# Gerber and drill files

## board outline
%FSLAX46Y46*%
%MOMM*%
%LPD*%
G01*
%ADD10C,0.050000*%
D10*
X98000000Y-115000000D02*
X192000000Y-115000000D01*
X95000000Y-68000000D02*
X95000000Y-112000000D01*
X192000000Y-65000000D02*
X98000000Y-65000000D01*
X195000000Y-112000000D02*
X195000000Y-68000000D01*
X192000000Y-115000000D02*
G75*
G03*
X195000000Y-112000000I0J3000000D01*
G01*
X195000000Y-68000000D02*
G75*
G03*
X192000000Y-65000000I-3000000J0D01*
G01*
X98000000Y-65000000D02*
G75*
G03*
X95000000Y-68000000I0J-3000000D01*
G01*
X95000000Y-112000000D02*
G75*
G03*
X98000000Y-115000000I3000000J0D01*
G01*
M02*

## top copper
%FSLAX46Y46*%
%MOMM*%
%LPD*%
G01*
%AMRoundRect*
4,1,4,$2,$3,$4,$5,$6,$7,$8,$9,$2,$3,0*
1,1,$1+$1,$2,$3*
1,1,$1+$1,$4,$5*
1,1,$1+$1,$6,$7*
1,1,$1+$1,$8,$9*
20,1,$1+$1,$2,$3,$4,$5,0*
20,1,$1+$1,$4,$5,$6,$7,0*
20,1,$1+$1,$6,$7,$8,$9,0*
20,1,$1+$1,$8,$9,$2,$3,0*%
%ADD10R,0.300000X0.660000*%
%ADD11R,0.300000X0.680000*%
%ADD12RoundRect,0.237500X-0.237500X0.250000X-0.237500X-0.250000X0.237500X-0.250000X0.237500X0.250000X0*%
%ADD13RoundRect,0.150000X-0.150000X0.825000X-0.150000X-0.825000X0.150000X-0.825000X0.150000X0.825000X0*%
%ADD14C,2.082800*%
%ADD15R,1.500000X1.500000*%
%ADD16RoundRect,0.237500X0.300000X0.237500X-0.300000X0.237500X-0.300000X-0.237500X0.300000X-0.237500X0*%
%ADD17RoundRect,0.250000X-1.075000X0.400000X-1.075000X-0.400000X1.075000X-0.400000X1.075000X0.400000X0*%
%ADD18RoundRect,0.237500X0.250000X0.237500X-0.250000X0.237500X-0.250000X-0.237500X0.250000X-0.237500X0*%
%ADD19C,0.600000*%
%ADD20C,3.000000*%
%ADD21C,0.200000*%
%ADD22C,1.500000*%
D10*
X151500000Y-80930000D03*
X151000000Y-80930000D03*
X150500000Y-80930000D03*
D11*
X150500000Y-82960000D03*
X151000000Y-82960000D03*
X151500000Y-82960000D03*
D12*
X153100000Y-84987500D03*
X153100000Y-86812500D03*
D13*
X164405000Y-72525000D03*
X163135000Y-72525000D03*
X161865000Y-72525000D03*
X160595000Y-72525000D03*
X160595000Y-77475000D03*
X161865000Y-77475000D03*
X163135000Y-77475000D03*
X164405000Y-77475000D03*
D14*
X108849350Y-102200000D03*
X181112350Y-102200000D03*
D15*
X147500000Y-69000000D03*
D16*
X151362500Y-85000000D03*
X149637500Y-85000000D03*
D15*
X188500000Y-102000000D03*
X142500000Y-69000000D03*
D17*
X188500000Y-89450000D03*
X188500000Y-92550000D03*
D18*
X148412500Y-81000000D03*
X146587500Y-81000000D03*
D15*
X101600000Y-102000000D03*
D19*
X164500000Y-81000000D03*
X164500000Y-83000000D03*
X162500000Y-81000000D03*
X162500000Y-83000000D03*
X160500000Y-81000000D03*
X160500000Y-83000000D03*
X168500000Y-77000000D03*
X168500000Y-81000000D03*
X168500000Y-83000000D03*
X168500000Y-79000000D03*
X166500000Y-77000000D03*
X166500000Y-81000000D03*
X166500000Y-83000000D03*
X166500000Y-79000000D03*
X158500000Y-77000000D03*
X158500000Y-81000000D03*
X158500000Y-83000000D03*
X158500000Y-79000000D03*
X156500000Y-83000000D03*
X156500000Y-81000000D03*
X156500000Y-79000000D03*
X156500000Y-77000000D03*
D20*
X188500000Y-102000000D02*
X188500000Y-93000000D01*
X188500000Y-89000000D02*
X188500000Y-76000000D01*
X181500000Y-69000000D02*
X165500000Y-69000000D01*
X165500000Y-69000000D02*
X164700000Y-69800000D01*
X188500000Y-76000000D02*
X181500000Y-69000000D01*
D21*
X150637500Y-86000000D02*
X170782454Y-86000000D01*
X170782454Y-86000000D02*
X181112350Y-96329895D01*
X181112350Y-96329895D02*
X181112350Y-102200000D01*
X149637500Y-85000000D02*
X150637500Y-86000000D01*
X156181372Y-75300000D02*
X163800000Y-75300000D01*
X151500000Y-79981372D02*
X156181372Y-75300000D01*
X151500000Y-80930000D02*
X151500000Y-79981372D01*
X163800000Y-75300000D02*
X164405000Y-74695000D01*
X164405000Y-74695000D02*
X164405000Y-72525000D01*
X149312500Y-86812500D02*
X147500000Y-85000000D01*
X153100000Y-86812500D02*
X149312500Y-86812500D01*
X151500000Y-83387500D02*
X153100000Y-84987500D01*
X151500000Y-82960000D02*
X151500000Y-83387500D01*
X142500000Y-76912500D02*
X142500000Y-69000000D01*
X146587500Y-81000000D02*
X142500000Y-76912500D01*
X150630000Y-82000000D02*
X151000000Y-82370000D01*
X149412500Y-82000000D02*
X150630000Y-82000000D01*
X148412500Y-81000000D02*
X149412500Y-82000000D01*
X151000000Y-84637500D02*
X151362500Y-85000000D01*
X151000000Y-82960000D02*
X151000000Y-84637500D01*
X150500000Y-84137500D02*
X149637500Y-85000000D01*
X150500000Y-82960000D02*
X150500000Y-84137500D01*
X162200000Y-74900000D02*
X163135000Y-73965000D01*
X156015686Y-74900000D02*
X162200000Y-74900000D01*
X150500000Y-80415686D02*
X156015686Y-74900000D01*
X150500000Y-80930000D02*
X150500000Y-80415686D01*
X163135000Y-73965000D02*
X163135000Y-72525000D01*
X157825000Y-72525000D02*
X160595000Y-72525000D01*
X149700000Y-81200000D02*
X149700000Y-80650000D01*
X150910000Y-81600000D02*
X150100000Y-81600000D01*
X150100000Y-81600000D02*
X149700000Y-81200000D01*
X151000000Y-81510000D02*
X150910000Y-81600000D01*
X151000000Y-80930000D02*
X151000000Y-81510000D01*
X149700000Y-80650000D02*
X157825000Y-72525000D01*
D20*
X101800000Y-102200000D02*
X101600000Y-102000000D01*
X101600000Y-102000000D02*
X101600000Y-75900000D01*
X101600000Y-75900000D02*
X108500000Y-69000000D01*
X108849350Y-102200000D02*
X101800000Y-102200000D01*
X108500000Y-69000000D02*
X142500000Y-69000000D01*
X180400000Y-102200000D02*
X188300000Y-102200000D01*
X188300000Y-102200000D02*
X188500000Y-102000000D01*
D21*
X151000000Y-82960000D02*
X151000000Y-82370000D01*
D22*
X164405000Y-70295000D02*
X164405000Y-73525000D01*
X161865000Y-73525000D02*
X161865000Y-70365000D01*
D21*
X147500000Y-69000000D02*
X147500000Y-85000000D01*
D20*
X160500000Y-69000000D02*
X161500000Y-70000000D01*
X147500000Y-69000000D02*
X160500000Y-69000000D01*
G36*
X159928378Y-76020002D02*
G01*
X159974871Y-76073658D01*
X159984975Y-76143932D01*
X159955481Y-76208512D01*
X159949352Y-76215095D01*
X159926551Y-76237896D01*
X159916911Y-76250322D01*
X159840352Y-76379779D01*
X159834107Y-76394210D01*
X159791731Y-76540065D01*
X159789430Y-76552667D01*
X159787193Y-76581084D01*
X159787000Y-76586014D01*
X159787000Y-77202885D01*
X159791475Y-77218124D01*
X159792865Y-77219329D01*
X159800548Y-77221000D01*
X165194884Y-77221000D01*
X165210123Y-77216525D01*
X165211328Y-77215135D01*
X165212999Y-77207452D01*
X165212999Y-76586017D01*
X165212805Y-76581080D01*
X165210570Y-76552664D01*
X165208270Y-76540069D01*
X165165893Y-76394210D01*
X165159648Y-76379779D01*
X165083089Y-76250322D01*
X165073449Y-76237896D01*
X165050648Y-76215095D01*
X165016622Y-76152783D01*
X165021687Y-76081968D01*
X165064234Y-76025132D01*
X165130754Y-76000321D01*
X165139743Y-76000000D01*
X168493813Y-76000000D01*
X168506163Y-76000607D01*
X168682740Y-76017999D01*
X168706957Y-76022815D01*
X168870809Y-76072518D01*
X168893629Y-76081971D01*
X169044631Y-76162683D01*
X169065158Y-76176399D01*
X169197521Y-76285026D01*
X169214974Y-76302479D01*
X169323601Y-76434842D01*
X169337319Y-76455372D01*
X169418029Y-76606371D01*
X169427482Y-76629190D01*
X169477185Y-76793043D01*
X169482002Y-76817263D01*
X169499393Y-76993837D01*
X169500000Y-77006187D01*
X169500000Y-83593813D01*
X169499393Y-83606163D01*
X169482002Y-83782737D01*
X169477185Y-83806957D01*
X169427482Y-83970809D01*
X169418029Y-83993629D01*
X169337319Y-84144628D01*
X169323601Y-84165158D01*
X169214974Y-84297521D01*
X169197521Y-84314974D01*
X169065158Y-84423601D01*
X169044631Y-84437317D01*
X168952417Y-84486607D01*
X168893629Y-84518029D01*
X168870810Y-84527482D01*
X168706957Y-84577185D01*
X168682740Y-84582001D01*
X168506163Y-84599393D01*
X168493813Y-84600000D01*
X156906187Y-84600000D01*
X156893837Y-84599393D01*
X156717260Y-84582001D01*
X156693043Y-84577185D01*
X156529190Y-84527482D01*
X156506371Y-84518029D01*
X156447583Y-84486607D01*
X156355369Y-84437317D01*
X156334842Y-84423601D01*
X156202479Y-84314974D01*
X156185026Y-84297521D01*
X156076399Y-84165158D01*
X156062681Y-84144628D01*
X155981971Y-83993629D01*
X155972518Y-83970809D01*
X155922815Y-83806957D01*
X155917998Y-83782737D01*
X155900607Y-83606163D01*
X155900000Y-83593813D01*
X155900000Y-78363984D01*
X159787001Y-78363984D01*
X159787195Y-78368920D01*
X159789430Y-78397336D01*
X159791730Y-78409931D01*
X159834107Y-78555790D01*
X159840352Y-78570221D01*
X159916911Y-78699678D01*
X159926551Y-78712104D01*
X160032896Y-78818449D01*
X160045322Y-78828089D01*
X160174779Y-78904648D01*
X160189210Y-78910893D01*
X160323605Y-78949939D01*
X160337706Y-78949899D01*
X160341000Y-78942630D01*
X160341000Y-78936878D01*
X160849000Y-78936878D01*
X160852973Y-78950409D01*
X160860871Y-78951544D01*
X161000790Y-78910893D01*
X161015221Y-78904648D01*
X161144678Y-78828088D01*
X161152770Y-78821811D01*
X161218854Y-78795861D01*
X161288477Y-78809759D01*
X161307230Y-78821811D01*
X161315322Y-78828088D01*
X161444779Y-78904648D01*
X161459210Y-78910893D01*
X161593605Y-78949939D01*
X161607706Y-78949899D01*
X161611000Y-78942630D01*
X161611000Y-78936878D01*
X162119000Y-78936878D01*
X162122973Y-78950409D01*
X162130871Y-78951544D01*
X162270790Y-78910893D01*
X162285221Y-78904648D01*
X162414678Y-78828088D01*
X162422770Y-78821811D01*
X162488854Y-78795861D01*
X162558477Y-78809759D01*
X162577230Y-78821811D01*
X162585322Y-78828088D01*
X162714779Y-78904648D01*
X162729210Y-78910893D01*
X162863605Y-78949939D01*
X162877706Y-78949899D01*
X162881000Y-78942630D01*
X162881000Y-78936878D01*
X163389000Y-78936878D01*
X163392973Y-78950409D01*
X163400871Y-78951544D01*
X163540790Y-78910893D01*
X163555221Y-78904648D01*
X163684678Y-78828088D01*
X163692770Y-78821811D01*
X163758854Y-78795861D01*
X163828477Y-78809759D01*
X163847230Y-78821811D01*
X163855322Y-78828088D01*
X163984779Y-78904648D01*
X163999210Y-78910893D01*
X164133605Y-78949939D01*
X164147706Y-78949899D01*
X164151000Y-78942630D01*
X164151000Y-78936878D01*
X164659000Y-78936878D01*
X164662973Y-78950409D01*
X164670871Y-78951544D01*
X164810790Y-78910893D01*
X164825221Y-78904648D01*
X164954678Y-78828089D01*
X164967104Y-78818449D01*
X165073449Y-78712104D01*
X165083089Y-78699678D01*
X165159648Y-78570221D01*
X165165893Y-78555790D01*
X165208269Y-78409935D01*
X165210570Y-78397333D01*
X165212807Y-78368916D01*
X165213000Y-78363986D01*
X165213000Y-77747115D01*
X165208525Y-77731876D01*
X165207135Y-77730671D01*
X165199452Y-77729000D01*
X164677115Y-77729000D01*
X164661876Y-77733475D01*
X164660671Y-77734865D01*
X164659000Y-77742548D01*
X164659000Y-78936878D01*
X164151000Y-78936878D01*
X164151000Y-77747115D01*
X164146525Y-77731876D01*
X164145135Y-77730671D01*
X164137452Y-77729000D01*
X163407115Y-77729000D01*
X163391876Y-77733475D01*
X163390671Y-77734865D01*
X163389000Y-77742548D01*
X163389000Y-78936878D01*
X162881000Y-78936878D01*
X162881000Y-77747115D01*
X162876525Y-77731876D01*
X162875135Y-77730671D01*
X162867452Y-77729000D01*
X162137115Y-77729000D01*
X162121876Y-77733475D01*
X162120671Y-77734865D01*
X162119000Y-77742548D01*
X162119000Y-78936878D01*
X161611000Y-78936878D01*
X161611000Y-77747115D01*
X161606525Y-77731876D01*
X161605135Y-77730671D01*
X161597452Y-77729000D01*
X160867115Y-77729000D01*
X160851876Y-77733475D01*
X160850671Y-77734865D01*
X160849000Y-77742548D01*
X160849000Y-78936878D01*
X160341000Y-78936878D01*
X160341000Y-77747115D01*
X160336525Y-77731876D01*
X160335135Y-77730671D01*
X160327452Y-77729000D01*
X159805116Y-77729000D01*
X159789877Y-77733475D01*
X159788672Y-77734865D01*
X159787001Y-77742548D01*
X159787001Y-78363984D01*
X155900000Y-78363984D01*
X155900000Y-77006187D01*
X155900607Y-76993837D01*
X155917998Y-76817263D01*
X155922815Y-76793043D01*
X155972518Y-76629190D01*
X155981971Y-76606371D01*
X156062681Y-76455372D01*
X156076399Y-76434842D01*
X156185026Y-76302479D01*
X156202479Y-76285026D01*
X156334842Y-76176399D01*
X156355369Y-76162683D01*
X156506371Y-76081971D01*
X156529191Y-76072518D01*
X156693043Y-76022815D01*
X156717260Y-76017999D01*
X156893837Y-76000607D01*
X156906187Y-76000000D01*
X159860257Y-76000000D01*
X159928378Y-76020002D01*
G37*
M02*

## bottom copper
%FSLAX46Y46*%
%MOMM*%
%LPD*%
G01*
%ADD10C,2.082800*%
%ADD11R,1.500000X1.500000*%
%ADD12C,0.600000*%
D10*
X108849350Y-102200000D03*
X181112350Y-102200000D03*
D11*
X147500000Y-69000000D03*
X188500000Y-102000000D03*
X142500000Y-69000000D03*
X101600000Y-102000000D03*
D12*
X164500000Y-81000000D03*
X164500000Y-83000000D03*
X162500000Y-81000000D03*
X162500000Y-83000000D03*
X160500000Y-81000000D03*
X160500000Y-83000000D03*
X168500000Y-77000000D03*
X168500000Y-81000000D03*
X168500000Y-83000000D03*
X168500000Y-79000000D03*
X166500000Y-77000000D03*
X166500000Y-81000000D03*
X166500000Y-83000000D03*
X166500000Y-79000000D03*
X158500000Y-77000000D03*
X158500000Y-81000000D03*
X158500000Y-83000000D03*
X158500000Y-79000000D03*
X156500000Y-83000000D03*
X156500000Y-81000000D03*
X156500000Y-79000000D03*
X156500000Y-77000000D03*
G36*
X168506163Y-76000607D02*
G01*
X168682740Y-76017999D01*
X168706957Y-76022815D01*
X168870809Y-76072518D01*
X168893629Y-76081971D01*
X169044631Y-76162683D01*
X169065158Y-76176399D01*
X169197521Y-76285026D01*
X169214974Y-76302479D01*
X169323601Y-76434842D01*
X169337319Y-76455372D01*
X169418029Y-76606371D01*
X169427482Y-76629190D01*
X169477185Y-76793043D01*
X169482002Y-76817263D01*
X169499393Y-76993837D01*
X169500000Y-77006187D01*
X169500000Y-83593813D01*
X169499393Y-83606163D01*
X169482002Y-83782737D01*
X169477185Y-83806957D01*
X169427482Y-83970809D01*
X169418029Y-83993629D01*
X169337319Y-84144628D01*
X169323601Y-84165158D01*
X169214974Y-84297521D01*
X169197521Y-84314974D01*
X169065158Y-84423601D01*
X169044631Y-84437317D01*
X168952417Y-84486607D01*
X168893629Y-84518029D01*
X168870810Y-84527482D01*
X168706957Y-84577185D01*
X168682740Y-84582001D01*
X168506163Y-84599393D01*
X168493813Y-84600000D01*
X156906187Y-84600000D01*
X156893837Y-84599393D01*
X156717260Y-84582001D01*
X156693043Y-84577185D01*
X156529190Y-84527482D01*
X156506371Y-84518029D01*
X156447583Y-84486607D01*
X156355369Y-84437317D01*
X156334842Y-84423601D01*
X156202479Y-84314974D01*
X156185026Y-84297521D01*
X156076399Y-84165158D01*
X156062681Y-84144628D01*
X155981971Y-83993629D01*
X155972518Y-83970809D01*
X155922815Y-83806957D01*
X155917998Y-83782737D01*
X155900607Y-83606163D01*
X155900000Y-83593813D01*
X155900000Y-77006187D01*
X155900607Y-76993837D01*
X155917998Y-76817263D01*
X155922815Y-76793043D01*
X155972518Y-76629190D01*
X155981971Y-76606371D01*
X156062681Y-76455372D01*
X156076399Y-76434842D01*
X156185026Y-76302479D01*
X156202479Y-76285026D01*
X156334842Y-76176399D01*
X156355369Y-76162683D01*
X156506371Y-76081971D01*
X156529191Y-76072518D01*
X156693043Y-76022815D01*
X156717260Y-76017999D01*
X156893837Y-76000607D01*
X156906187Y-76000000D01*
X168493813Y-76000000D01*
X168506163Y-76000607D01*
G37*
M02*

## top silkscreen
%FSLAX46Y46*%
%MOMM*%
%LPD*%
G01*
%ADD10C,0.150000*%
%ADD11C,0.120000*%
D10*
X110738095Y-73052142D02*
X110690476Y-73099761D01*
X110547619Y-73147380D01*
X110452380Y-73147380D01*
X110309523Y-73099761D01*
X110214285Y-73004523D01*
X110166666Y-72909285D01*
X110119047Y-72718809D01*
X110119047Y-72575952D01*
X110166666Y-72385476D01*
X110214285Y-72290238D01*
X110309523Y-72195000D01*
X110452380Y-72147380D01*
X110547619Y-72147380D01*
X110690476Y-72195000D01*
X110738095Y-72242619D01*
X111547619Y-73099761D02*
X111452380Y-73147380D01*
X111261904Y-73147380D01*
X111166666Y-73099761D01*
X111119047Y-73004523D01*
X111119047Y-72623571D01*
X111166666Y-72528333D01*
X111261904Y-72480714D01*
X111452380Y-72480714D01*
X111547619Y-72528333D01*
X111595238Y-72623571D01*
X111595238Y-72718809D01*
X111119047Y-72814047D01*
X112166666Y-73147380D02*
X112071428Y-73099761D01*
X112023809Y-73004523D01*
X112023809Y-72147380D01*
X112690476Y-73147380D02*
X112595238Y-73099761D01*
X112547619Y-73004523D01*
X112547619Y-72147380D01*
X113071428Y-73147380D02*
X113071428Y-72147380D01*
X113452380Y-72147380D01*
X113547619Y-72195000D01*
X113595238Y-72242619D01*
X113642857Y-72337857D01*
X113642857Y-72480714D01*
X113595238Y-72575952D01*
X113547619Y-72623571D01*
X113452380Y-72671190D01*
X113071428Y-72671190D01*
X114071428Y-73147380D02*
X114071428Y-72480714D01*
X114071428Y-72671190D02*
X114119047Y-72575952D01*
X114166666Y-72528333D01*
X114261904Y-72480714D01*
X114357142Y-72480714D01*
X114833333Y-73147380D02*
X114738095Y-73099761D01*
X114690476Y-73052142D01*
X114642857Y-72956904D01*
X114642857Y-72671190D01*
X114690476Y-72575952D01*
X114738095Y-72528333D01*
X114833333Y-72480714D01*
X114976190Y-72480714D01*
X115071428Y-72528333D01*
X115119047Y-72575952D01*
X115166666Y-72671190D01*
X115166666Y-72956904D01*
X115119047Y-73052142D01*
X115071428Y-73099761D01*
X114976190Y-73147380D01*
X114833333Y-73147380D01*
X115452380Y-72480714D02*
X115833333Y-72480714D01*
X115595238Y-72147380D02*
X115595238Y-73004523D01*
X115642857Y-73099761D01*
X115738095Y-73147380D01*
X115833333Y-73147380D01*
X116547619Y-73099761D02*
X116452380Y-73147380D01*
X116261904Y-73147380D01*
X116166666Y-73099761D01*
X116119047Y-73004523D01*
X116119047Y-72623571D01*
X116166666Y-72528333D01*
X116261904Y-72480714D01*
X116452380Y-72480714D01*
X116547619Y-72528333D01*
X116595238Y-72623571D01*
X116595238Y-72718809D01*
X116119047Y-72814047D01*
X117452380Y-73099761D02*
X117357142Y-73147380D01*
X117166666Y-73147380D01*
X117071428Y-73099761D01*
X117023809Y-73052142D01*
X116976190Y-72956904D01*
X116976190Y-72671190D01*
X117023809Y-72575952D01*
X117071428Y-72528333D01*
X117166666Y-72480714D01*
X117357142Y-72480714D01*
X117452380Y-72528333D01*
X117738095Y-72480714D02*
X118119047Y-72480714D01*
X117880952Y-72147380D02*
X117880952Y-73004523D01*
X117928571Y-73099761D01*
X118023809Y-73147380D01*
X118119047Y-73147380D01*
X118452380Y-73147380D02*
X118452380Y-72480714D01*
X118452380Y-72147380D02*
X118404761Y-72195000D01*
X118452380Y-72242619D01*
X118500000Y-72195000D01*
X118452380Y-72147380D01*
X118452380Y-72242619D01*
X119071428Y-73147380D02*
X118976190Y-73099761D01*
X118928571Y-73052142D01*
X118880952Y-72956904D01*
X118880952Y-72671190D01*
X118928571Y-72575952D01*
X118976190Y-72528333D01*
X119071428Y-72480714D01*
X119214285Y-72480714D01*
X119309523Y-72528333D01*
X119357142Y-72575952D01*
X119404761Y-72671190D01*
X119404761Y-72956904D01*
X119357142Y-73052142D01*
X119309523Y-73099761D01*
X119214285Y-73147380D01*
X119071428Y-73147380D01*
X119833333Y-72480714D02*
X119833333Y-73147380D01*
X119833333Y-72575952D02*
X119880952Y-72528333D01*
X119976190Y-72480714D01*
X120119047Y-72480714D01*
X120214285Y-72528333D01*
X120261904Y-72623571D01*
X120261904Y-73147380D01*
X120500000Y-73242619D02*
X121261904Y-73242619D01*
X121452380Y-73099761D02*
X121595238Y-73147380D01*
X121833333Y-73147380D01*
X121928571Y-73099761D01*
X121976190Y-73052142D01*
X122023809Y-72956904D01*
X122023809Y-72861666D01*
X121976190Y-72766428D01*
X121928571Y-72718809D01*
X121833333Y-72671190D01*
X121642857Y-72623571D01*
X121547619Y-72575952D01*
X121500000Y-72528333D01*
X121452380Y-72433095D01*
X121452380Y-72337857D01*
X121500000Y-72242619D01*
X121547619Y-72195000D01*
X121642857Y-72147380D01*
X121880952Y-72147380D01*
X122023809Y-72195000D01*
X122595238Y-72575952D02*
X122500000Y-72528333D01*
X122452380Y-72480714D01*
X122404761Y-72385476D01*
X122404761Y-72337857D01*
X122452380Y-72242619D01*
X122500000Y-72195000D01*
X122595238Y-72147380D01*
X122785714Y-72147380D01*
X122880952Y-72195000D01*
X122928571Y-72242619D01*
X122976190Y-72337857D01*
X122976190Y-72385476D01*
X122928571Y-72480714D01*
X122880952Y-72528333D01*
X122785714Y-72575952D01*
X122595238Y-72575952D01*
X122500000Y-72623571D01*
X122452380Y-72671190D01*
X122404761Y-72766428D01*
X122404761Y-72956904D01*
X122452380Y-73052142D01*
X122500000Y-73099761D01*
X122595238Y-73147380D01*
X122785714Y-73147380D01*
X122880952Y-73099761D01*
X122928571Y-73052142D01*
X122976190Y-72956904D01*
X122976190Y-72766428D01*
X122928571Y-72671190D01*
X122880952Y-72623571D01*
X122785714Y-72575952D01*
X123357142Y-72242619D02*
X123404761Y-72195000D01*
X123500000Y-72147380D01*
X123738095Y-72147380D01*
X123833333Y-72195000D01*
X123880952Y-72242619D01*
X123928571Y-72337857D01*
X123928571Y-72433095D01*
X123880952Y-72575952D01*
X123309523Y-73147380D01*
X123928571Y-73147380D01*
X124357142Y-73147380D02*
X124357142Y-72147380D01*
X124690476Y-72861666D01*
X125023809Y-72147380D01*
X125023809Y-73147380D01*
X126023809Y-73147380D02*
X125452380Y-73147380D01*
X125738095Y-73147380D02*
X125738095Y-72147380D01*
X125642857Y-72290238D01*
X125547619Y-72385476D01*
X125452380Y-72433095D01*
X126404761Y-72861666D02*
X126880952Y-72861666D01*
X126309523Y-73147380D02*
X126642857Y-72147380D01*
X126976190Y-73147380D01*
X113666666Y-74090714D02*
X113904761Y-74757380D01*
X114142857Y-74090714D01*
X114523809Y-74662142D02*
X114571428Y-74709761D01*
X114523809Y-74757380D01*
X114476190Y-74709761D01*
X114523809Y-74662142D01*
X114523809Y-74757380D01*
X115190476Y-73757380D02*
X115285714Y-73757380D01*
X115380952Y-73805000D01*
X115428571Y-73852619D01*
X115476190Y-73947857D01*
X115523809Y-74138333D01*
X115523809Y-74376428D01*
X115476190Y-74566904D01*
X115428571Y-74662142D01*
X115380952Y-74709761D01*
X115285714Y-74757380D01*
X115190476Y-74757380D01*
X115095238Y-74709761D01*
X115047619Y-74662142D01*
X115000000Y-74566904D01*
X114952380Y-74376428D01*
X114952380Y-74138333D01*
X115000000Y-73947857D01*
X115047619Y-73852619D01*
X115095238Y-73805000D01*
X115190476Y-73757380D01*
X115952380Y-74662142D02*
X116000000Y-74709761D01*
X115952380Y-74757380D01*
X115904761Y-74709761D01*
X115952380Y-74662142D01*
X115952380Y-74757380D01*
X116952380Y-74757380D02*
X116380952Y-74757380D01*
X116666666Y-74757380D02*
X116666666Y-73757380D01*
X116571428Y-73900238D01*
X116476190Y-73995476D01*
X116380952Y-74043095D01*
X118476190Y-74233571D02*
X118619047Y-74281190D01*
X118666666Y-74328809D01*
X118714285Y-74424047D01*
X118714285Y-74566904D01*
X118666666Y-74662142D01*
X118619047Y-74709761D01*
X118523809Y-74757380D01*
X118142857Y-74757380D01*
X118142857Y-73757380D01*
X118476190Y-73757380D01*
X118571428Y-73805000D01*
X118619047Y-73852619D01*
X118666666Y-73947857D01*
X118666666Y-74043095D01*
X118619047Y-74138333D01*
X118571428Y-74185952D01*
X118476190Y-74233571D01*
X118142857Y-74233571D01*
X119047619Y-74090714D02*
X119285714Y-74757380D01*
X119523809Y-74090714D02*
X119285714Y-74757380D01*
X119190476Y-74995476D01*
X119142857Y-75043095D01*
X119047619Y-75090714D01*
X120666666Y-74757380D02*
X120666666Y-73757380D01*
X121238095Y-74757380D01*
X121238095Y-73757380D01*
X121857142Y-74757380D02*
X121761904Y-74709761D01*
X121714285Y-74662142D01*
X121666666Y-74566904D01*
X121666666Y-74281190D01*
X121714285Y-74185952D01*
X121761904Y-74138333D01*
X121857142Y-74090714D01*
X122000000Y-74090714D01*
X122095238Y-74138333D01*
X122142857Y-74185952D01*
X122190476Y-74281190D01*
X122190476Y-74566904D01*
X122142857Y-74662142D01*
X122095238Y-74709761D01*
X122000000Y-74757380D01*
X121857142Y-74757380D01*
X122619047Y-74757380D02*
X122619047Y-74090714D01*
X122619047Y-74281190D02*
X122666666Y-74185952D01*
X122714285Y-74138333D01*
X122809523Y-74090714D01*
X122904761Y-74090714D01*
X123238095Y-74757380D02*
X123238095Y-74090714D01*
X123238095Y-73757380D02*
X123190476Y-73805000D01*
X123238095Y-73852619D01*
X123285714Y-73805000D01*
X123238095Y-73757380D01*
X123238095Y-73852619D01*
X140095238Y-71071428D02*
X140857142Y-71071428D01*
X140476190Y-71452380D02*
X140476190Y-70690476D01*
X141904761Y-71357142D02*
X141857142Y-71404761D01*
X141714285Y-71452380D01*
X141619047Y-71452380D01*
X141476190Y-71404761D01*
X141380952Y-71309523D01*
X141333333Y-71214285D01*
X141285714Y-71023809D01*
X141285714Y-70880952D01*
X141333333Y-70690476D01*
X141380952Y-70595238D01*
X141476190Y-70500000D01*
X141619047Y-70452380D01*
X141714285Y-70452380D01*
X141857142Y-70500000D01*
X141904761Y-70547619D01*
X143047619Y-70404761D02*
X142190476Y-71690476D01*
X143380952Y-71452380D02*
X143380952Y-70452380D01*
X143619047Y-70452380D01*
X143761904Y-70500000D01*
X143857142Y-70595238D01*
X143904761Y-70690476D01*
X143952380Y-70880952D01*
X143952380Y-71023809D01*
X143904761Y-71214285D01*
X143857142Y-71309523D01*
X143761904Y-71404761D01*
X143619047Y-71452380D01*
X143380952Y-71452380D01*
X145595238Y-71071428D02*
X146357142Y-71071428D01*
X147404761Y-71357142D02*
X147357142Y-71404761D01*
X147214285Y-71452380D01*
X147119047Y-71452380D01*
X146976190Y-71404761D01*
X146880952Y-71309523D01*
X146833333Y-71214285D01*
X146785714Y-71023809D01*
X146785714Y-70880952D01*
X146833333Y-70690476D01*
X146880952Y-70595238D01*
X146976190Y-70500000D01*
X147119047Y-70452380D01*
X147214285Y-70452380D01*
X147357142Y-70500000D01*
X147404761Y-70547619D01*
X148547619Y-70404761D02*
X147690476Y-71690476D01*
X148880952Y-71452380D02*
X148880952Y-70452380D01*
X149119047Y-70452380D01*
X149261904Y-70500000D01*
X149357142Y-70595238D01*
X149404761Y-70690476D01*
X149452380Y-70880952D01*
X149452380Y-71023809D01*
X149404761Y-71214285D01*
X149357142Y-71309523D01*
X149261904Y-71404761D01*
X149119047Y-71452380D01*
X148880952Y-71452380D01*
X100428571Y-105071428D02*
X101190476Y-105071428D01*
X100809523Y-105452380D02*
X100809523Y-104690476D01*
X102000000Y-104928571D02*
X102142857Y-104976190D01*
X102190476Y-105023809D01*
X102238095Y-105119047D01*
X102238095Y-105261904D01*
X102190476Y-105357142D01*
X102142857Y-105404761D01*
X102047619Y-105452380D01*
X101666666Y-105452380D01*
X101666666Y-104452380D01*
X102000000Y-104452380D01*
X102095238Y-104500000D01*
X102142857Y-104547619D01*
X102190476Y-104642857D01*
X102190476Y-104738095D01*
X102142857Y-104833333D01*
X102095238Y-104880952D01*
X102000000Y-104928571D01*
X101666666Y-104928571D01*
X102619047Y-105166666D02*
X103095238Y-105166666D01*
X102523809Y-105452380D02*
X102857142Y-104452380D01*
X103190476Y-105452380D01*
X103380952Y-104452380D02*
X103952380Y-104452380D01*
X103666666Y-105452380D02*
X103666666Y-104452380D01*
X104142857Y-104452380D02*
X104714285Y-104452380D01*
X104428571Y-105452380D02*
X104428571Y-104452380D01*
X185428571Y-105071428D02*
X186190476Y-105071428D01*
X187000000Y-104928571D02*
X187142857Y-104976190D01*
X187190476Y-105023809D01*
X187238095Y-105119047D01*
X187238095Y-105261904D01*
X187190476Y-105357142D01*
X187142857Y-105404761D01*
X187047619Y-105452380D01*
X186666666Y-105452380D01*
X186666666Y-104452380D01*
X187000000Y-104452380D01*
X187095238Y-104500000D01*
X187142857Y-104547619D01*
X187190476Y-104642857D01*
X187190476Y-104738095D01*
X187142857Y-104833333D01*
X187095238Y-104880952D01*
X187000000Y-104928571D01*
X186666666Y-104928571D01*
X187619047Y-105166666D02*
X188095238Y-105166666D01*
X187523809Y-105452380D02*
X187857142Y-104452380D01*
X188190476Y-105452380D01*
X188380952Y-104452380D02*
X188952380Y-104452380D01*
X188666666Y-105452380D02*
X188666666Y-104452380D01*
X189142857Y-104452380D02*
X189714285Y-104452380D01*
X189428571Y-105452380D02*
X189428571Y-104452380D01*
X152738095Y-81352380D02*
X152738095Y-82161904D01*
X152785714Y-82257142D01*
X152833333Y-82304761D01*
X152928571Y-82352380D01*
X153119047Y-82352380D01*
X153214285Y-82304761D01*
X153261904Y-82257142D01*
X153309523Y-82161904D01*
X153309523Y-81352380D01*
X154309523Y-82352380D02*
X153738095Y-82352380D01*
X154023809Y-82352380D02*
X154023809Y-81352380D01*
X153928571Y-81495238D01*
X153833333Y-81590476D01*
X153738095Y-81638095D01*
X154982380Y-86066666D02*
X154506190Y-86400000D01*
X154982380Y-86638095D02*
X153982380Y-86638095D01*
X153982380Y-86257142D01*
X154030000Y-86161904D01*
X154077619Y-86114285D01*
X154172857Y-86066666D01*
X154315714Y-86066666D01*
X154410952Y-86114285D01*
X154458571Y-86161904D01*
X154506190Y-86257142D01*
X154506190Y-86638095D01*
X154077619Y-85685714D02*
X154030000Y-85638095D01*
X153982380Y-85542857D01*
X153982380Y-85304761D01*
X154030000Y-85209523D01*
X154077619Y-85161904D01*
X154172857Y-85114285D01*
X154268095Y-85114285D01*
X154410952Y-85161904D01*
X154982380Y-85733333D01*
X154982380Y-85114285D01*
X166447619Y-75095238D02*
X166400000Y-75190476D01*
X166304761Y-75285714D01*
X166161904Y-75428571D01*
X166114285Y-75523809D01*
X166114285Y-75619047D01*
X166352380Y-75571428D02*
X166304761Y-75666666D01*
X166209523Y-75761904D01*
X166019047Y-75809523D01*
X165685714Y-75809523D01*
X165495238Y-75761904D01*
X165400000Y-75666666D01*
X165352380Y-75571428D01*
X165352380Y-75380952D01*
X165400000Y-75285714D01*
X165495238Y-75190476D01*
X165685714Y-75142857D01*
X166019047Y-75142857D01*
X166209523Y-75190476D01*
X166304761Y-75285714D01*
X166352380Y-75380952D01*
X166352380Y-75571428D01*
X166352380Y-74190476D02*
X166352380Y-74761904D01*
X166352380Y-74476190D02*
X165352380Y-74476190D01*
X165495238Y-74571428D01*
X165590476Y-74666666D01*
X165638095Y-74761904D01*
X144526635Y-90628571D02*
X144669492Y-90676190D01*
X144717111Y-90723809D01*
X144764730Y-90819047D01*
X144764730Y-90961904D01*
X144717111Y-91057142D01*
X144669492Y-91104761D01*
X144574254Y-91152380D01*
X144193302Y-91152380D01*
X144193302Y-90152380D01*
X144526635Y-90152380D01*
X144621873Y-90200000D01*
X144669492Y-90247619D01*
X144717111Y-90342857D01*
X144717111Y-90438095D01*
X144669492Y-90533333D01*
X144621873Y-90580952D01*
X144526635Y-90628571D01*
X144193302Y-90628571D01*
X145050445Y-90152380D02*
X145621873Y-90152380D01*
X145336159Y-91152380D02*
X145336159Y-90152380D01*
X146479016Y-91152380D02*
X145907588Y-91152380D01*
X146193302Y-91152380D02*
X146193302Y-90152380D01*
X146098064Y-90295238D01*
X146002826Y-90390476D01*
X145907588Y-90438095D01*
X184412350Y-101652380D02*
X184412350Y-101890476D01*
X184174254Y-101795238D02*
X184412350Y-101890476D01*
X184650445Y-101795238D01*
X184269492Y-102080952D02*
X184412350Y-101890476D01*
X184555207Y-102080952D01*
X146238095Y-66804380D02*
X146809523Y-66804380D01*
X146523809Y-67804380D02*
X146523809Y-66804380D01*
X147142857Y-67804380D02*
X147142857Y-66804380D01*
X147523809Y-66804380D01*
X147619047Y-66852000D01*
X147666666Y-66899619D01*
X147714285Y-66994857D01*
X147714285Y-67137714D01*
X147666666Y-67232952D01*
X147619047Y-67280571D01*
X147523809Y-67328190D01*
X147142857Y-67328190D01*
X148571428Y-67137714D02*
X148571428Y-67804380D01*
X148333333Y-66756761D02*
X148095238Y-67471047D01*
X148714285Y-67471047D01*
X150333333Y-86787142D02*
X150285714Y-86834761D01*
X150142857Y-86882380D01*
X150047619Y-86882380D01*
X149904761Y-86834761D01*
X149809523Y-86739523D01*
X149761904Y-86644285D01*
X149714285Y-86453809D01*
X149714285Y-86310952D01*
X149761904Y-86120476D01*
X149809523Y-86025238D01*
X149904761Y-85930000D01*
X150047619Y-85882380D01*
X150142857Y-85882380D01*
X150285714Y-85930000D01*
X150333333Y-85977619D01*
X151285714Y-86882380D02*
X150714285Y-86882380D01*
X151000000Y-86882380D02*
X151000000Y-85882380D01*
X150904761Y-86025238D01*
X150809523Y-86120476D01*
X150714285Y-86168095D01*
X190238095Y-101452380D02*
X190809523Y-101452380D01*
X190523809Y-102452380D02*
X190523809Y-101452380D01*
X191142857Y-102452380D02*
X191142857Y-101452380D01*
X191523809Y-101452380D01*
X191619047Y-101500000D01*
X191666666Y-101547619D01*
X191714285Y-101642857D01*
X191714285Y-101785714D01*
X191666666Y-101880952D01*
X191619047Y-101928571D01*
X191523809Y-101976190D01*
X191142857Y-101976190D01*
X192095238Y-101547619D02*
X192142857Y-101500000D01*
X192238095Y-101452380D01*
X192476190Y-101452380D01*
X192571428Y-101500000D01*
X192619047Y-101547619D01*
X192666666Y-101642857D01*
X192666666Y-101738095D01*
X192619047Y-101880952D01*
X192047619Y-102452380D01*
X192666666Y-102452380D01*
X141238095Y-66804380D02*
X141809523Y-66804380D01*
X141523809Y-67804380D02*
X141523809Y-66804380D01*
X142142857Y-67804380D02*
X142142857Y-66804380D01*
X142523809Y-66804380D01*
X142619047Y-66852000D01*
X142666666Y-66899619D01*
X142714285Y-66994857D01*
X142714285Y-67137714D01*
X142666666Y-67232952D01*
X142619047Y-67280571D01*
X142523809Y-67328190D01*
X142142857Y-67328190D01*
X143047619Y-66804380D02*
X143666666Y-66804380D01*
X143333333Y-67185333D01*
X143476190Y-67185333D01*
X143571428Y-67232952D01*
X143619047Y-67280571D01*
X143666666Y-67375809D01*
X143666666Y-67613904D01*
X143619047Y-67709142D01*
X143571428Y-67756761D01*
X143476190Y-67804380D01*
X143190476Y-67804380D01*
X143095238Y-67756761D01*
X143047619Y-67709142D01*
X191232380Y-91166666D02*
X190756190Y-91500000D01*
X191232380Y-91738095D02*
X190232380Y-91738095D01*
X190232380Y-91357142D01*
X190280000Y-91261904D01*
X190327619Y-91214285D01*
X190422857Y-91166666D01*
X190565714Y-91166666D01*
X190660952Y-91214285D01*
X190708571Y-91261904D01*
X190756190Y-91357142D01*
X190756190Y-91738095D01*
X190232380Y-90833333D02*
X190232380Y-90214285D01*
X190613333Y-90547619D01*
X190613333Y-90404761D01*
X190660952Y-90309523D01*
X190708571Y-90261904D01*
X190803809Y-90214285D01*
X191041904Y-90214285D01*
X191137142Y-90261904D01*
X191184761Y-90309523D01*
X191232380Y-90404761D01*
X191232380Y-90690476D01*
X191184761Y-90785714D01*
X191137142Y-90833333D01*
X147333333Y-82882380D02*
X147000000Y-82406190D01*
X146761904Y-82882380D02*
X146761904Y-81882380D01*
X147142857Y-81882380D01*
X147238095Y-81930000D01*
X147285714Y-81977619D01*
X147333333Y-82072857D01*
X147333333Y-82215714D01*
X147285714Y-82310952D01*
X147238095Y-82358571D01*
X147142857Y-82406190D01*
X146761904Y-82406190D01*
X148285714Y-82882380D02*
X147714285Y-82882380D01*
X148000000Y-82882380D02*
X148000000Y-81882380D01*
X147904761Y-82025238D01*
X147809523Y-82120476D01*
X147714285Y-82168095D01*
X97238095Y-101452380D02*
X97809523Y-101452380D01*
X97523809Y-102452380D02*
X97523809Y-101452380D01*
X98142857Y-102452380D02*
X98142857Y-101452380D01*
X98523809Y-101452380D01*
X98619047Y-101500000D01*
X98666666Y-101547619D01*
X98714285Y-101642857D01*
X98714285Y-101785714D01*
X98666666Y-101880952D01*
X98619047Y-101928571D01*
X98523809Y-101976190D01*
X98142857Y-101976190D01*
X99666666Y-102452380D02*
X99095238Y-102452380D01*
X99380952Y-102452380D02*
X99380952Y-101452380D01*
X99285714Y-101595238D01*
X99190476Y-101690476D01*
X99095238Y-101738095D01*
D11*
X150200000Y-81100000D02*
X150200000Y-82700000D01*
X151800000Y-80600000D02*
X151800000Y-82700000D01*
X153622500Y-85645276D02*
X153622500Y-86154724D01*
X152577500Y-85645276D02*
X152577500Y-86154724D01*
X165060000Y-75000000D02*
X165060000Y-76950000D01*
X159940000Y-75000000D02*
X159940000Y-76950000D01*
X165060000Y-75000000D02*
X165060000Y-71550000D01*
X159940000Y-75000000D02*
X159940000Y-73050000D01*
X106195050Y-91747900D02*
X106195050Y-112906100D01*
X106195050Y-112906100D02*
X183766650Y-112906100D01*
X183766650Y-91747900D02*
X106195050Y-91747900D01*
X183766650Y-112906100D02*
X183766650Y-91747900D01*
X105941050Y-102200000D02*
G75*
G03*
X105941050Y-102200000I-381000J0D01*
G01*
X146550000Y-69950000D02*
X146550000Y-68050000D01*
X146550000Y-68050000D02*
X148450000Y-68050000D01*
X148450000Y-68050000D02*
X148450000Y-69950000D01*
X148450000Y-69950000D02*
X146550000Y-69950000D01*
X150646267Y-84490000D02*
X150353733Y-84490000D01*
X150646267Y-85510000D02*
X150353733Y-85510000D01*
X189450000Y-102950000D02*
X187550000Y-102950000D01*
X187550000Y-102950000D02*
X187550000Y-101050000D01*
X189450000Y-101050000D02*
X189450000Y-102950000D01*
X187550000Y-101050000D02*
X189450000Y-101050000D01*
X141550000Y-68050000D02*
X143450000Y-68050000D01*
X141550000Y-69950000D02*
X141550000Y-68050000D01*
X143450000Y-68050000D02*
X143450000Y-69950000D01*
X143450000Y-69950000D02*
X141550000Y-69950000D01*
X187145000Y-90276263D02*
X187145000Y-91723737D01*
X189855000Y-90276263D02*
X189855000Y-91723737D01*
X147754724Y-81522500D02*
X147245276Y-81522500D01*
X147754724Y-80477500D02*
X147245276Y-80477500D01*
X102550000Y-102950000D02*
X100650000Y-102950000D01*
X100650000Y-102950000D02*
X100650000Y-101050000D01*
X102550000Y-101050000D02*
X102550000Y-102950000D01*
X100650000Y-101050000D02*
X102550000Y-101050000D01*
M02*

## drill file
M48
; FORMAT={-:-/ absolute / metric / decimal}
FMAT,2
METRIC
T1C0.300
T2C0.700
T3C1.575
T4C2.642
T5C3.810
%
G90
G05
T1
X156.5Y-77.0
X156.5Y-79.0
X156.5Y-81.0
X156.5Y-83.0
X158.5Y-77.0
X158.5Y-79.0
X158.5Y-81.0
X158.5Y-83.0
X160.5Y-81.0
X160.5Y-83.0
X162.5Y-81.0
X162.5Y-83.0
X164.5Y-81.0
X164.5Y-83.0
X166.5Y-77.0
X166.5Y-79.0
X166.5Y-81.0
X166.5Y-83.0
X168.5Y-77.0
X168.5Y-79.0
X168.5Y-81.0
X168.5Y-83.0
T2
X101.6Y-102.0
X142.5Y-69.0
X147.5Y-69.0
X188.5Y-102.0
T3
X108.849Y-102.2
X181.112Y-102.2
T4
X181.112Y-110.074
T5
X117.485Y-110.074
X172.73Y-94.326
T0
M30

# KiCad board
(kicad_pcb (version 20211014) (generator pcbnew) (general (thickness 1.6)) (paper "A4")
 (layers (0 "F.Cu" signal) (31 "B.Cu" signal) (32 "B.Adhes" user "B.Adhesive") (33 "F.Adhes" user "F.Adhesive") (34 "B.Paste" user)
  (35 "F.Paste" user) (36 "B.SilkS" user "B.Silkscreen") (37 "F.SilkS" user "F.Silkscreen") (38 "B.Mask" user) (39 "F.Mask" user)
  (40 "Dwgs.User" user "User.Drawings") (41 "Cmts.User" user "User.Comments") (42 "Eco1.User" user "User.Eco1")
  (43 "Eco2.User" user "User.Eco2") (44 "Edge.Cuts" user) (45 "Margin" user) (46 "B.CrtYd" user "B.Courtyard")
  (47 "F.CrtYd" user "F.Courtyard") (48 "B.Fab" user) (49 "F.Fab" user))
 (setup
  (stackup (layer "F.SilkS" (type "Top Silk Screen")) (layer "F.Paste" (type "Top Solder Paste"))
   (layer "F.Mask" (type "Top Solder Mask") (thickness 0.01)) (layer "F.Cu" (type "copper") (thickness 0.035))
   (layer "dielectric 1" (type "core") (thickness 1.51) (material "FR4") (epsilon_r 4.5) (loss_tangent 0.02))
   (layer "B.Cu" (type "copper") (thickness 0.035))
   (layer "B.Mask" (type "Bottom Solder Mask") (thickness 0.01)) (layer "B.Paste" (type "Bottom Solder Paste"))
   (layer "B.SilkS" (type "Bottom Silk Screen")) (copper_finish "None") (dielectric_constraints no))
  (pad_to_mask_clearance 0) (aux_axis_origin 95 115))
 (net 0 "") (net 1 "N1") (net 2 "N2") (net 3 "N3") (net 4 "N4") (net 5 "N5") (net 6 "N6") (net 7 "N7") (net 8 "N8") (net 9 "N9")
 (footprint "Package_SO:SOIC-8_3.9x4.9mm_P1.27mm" (layer "F.Cu") (at 162.5 75 -90)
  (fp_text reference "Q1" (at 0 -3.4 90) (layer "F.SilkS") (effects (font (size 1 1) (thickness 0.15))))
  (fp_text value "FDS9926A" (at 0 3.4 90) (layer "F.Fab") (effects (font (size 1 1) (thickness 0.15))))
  (fp_line (start 0 -2.56) (end 1.95 -2.56) (layer "F.SilkS") (width 0.12))
  (fp_line (start 0 2.56) (end 1.95 2.56) (layer "F.SilkS") (width 0.12))
  (fp_line (start 0 -2.56) (end -3.45 -2.56) (layer "F.SilkS") (width 0.12))
  (fp_line (start 0 2.56) (end -1.95 2.56) (layer "F.SilkS") (width 0.12))
  (pad "1" smd roundrect (at -2.475 -1.905 270) (size 1.95 0.6) (layers "F.Cu" "F.Paste" "F.Mask") (roundrect_rratio 0.25) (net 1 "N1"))
  (pad "2" smd roundrect (at -2.475 -0.635 270) (size 1.95 0.6) (layers "F.Cu" "F.Paste" "F.Mask") (roundrect_rratio 0.25) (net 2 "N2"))
  (pad "3" smd roundrect (at -2.475 0.635 270) (size 1.95 0.6) (layers "F.Cu" "F.Paste" "F.Mask") (roundrect_rratio 0.25) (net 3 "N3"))
  (pad "4" smd roundrect (at -2.475 1.905 270) (size 1.95 0.6) (layers "F.Cu" "F.Paste" "F.Mask") (roundrect_rratio 0.25) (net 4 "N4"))
  (pad "5" smd roundrect (at 2.475 1.905 270) (size 1.95 0.6) (layers "F.Cu" "F.Paste" "F.Mask") (roundrect_rratio 0.25) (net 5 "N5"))
  (pad "6" smd roundrect (at 2.475 0.635 270) (size 1.95 0.6) (layers "F.Cu" "F.Paste" "F.Mask") (roundrect_rratio 0.25) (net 5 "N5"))
  (pad "7" smd roundrect (at 2.475 -0.635 270) (size 1.95 0.6) (layers "F.Cu" "F.Paste" "F.Mask") (roundrect_rratio 0.25) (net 5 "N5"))
  (pad "8" smd roundrect (at 2.475 -1.905 270) (size 1.95 0.6) (layers "F.Cu" "F.Paste" "F.Mask") (roundrect_rratio 0.25) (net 5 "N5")))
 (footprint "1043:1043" (layer "F.Cu") (at 181.11235 102.2)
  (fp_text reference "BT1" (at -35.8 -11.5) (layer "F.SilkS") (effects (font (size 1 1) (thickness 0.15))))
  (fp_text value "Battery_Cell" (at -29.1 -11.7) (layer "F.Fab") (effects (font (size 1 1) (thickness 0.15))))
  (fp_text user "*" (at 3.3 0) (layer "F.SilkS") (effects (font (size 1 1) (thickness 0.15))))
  (fp_line (start -74.9173 -10.4521) (end -74.9173 10.7061) (layer "F.SilkS") (width 0.12))
  (fp_line (start -74.9173 10.7061) (end 2.6543 10.7061) (layer "F.SilkS") (width 0.12))
  (fp_line (start 2.6543 -10.4521) (end -74.9173 -10.4521) (layer "F.SilkS") (width 0.12))
  (fp_line (start 2.6543 10.7061) (end 2.6543 -10.4521) (layer "F.SilkS") (width 0.12))
  (fp_circle (center -75.5523 0) (end -75.1713 0) (layer "F.SilkS") (width 0.12) (fill none))
  (pad "" np_thru_hole circle (at -8.382 -7.874) (size 3.81 3.81) (drill 3.81) (layers *.Cu *.Mask))
  (pad "" np_thru_hole circle (at -63.627 7.874) (size 3.81 3.81) (drill 3.81) (layers *.Cu *.Mask))
  (pad "" np_thru_hole circle (at 0 7.874) (size 2.6416 2.6416) (drill 2.6416) (layers *.Cu *.Mask))
  (pad "1" thru_hole circle (at -72.263 0) (size 2.0828 2.0828) (drill 1.5748) (layers *.Cu *.Mask) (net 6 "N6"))
  (pad "2" thru_hole circle (at 0 0) (size 2.0828 2.0828) (drill 1.5748) (layers *.Cu *.Mask) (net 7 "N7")))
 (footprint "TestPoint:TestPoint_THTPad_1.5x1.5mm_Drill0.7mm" (layer "F.Cu") (at 147.5 69)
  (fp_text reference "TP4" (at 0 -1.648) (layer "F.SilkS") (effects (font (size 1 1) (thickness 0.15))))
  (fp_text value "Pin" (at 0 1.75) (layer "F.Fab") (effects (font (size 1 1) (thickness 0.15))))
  (fp_line (start -0.95 0.95) (end -0.95 -0.95) (layer "F.SilkS") (width 0.12))
  (fp_line (start -0.95 -0.95) (end 0.95 -0.95) (layer "F.SilkS") (width 0.12))
  (fp_line (start 0.95 -0.95) (end 0.95 0.95) (layer "F.SilkS") (width 0.12))
  (fp_line (start 0.95 0.95) (end -0.95 0.95) (layer "F.SilkS") (width 0.12))
  (pad "1" thru_hole rect (at 0 0) (size 1.5 1.5) (drill 0.7) (layers *.Cu *.Mask) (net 3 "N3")))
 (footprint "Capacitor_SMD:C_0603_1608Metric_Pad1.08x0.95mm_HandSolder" (layer "F.Cu") (at 150.5 85 180)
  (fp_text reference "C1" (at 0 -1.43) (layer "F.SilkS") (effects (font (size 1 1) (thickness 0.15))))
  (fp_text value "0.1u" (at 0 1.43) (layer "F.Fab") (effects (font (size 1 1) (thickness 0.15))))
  (fp_line (start -0.146267 0.51) (end 0.146267 0.51) (layer "F.SilkS") (width 0.12))
  (fp_line (start -0.146267 -0.51) (end 0.146267 -0.51) (layer "F.SilkS") (width 0.12))
  (pad "1" smd roundrect (at -0.8625 0 180) (size 1.075 0.95) (layers "F.Cu" "F.Paste" "F.Mask") (roundrect_rratio 0.25) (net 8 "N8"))
  (pad "2" smd roundrect (at 0.8625 0 180) (size 1.075 0.95) (layers "F.Cu" "F.Paste" "F.Mask") (roundrect_rratio 0.25) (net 7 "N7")))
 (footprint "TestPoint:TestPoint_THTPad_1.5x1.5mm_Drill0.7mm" (layer "F.Cu") (at 188.5 102)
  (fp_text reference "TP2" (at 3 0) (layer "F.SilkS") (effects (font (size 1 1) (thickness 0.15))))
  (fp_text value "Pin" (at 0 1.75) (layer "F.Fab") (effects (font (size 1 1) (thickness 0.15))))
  (fp_line (start 0.95 0.95) (end -0.95 0.95) (layer "F.SilkS") (width 0.12))
  (fp_line (start -0.95 0.95) (end -0.95 -0.95) (layer "F.SilkS") (width 0.12))
  (fp_line (start 0.95 -0.95) (end 0.95 0.95) (layer "F.SilkS") (width 0.12))
  (fp_line (start -0.95 -0.95) (end 0.95 -0.95) (layer "F.SilkS") (width 0.12))
  (pad "1" thru_hole rect (at 0 0) (size 1.5 1.5) (drill 0.7) (layers *.Cu *.Mask) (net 7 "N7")))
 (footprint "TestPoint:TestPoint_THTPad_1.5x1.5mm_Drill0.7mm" (layer "F.Cu") (at 142.5 69)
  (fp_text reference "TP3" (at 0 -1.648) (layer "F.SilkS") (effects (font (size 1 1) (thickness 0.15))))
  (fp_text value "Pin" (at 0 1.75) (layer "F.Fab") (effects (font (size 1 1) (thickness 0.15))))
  (fp_line (start -0.95 -0.95) (end 0.95 -0.95) (layer "F.SilkS") (width 0.12))
  (fp_line (start -0.95 0.95) (end -0.95 -0.95) (layer "F.SilkS") (width 0.12))
  (fp_line (start 0.95 -0.95) (end 0.95 0.95) (layer "F.SilkS") (width 0.12))
  (fp_line (start 0.95 0.95) (end -0.95 0.95) (layer "F.SilkS") (width 0.12))
  (pad "1" thru_hole rect (at 0 0) (size 1.5 1.5) (drill 0.7) (layers *.Cu *.Mask) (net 6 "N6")))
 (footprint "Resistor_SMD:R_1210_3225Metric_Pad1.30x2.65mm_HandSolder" (layer "F.Cu") (at 188.5 91 -90)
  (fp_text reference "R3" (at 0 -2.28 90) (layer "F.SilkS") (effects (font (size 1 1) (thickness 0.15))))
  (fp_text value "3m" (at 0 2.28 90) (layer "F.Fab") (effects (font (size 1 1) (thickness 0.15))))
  (fp_line (start -0.723737 1.355) (end 0.723737 1.355) (layer "F.SilkS") (width 0.12))
  (fp_line (start -0.723737 -1.355) (end 0.723737 -1.355) (layer "F.SilkS") (width 0.12))
  (pad "1" smd roundrect (at -1.55 0 270) (size 1.3 2.65) (layers "F.Cu" "F.Paste" "F.Mask") (roundrect_rratio 0.1923076923) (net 1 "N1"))
  (pad "2" smd roundrect (at 1.55 0 270) (size 1.3 2.65) (layers "F.Cu" "F.Paste" "F.Mask") (roundrect_rratio 0.1923076923) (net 7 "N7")))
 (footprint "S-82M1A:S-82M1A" (layer "F.Cu") (at 151.5 81 180)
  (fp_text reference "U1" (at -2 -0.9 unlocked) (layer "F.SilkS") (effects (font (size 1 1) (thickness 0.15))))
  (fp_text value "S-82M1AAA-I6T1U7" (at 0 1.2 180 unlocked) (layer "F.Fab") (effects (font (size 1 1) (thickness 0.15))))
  (fp_line (start -0.3 0.4) (end -0.3 -1.7) (layer "F.SilkS") (width 0.12))
  (fp_line (start 1.3 -0.1) (end 1.3 -1.7) (layer "F.SilkS") (width 0.12))
  (pad "1" smd rect (at 0 0.07 270) (size 0.66 0.3) (layers "F.Cu" "F.Paste" "F.Mask") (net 1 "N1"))
  (pad "2" smd rect (at 0.5 0.07 270) (size 0.66 0.3) (layers "F.Cu" "F.Paste" "F.Mask") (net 4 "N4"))
  (pad "3" smd rect (at 1 0.07 270) (size 0.66 0.3) (layers "F.Cu" "F.Paste" "F.Mask") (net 2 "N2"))
  (pad "4" smd rect (at 1 -1.96 270) (size 0.68 0.3) (layers "F.Cu" "F.Paste" "F.Mask") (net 7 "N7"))
  (pad "5" smd rect (at 0.5 -1.96 270) (size 0.68 0.3) (layers "F.Cu" "F.Paste" "F.Mask") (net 8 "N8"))
  (pad "6" smd rect (at 0 -1.96 270) (size 0.68 0.3) (layers "F.Cu" "F.Paste" "F.Mask") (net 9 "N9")))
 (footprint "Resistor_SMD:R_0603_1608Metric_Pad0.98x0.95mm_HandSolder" (layer "F.Cu") (at 147.5 81 180)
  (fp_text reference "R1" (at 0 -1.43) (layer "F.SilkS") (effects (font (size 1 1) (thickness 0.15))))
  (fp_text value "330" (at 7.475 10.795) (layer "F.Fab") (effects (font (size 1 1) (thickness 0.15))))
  (fp_line (start -0.254724 -0.5225) (end 0.254724 -0.5225) (layer "F.SilkS") (width 0.12))
  (fp_line (start -0.254724 0.5225) (end 0.254724 0.5225) (layer "F.SilkS") (width 0.12))
  (pad "1" smd roundrect (at -0.9125 0 180) (size 0.975 0.95) (layers "F.Cu" "F.Paste" "F.Mask") (roundrect_rratio 0.25) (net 8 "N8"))
  (pad "2" smd roundrect (at 0.9125 0 180) (size 0.975 0.95) (layers "F.Cu" "F.Paste" "F.Mask") (roundrect_rratio 0.25) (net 6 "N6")))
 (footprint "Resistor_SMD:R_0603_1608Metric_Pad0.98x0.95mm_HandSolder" (layer "F.Cu") (at 153.1 85.9 -90)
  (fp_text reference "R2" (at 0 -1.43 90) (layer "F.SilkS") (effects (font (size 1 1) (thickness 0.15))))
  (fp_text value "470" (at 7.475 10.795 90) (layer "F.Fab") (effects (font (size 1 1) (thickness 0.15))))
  (fp_line (start -0.254724 -0.5225) (end 0.254724 -0.5225) (layer "F.SilkS") (width 0.12))
  (fp_line (start -0.254724 0.5225) (end 0.254724 0.5225) (layer "F.SilkS") (width 0.12))
  (pad "1" smd roundrect (at -0.9125 0 270) (size 0.975 0.95) (layers "F.Cu" "F.Paste" "F.Mask") (roundrect_rratio 0.25) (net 9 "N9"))
  (pad "2" smd roundrect (at 0.9125 0 270) (size 0.975 0.95) (layers "F.Cu" "F.Paste" "F.Mask") (roundrect_rratio 0.25) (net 3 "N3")))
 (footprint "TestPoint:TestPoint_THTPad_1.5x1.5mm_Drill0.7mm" (layer "F.Cu") (at 101.6 102)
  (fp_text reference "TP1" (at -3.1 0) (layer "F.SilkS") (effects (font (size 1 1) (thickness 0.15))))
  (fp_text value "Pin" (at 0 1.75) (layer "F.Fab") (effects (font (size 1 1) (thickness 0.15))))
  (fp_line (start 0.95 0.95) (end -0.95 0.95) (layer "F.SilkS") (width 0.12))
  (fp_line (start -0.95 0.95) (end -0.95 -0.95) (layer "F.SilkS") (width 0.12))
  (fp_line (start 0.95 -0.95) (end 0.95 0.95) (layer "F.SilkS") (width 0.12))
  (fp_line (start -0.95 -0.95) (end 0.95 -0.95) (layer "F.SilkS") (width 0.12))
  (pad "1" thru_hole rect (at 0 0) (size 1.5 1.5) (drill 0.7) (layers *.Cu *.Mask) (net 6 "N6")))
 (gr_arc (start 192 65) (mid 194.12132 65.87868) (end 195 68) (layer "Edge.Cuts") (width 0.05))
 (gr_arc (start 195 112) (mid 194.12132 114.12132) (end 192 115) (layer "Edge.Cuts") (width 0.05))
 (gr_line (start 195 112) (end 195 68) (layer "Edge.Cuts") (width 0.05))
 (gr_arc (start 95 68) (mid 95.87868 65.87868) (end 98 65) (layer "Edge.Cuts") (width 0.05))
 (gr_line (start 192 65) (end 98 65) (layer "Edge.Cuts") (width 0.05))
 (gr_line (start 98 115) (end 192 115) (layer "Edge.Cuts") (width 0.05))
 (gr_arc (start 98 115) (mid 95.87868 114.12132) (end 95 112) (layer "Edge.Cuts") (width 0.05))
 (gr_line (start 95 68) (end 95 112) (layer "Edge.Cuts") (width 0.05))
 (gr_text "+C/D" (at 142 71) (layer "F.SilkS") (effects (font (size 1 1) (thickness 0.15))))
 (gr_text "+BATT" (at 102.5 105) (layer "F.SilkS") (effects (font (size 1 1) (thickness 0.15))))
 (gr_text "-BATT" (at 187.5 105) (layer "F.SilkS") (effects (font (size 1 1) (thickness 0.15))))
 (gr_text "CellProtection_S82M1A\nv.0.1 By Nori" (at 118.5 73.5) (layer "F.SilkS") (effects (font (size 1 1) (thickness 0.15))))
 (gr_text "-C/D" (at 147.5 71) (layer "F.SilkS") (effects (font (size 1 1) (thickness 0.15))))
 (segment (start 142.5 76.9125) (end 142.5 69) (width 0.2) (layer "F.Cu") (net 6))
 (segment (start 101.8 102.2) (end 101.6 102) (width 3) (layer "F.Cu") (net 6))
 (segment (start 101.6 102) (end 101.6 75.9) (width 3) (layer "F.Cu") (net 6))
 (segment (start 101.6 75.9) (end 108.5 69) (width 3) (layer "F.Cu") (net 6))
 (segment (start 108.84935 102.2) (end 101.8 102.2) (width 3) (layer "F.Cu") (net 6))
 (segment (start 108.5 69) (end 142.5 69) (width 3) (layer "F.Cu") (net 6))
 (segment (start 146.5875 81) (end 142.5 76.9125) (width 0.2) (layer "F.Cu") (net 6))
 (segment (start 150.5 84.1375) (end 149.6375 85) (width 0.2) (layer "F.Cu") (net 7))
 (segment (start 170.782454 86) (end 181.11235 96.329895) (width 0.2) (layer "F.Cu") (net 7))
 (segment (start 180.4 102.2) (end 188.3 102.2) (width 3) (layer "F.Cu") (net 7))
 (segment (start 181.11235 96.329895) (end 181.11235 102.2) (width 0.2) (layer "F.Cu") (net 7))
 (segment (start 150.5 82.96) (end 150.5 84.1375) (width 0.2) (layer "F.Cu") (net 7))
 (segment (start 188.5 102) (end 188.5 93) (width 3) (layer "F.Cu") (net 7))
 (segment (start 188.3 102.2) (end 188.5 102) (width 3) (layer "F.Cu") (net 7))
 (segment (start 149.6375 85) (end 150.6375 86) (width 0.2) (layer "F.Cu") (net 7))
 (segment (start 150.6375 86) (end 170.782454 86) (width 0.2) (layer "F.Cu") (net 7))
 (segment (start 151 84.6375) (end 151.3625 85) (width 0.2) (layer "F.Cu") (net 8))
 (segment (start 151 82.96) (end 151 84.6375) (width 0.2) (layer "F.Cu") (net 8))
 (segment (start 149.4125 82) (end 150.63 82) (width 0.2) (layer "F.Cu") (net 8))
 (segment (start 150.63 82) (end 151 82.37) (width 0.2) (layer "F.Cu") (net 8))
 (segment (start 151 82.96) (end 151 82.37) (width 0.2) (layer "F.Cu") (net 8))
 (segment (start 148.4125 81) (end 149.4125 82) (width 0.2) (layer "F.Cu") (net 8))
 (segment (start 188.5 89) (end 188.5 76) (width 3) (layer "F.Cu") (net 1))
 (segment (start 163.8 75.3) (end 164.405 74.695) (width 0.2) (layer "F.Cu") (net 1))
 (segment (start 164.405 74.695) (end 164.405 72.525) (width 0.2) (layer "F.Cu") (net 1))
 (segment (start 181.5 69) (end 165.5 69) (width 3) (layer "F.Cu") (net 1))
 (segment (start 151.5 80.93) (end 151.5 79.981372) (width 0.2) (layer "F.Cu") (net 1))
 (segment (start 164.405 70.295) (end 164.405 73.525) (width 1.5) (layer "F.Cu") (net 1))
 (segment (start 151.5 79.981372) (end 156.181372 75.3) (width 0.2) (layer "F.Cu") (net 1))
 (segment (start 156.181372 75.3) (end 163.8 75.3) (width 0.2) (layer "F.Cu") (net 1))
 (segment (start 188.5 76) (end 181.5 69) (width 3) (layer "F.Cu") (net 1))
 (segment (start 165.5 69) (end 164.7 69.8) (width 3) (layer "F.Cu") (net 1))
 (segment (start 150.5 80.93) (end 150.5 80.415686) (width 0.2) (layer "F.Cu") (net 2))
 (segment (start 150.5 80.415686) (end 156.015686 74.9) (width 0.2) (layer "F.Cu") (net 2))
 (segment (start 163.135 73.965) (end 163.135 72.525) (width 0.2) (layer "F.Cu") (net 2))
 (segment (start 162.2 74.9) (end 163.135 73.965) (width 0.2) (layer "F.Cu") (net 2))
 (segment (start 156.015686 74.9) (end 162.2 74.9) (width 0.2) (layer "F.Cu") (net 2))
 (segment (start 149.3125 86.8125) (end 147.5 85) (width 0.2) (layer "F.Cu") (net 3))
 (segment (start 161.865 73.525) (end 161.865 70.365) (width 1.5) (layer "F.Cu") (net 3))
 (segment (start 153.1 86.8125) (end 149.3125 86.8125) (width 0.2) (layer "F.Cu") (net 3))
 (segment (start 147.5 69) (end 147.5 85) (width 0.2) (layer "F.Cu") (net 3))
 (segment (start 160.5 69) (end 161.5 70) (width 3) (layer "F.Cu") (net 3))
 (segment (start 147.5 69) (end 160.5 69) (width 3) (layer "F.Cu") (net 3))
 (segment (start 150.1 81.6) (end 149.7 81.2) (width 0.2) (layer "F.Cu") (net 4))
 (segment (start 150.91 81.6) (end 150.1 81.6) (width 0.2) (layer "F.Cu") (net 4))
 (segment (start 151 81.51) (end 150.91 81.6) (width 0.2) (layer "F.Cu") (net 4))
 (segment (start 149.7 80.65) (end 157.825 72.525) (width 0.2) (layer "F.Cu") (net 4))
 (segment (start 157.825 72.525) (end 160.595 72.525) (width 0.2) (layer "F.Cu") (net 4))
 (segment (start 149.7 81.2) (end 149.7 80.65) (width 0.2) (layer "F.Cu") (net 4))
 (segment (start 151 80.93) (end 151 81.51) (width 0.2) (layer "F.Cu") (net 4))
 (via (at 156.5 83) (size 0.6) (drill 0.3) (layers "F.Cu" "B.Cu") (free) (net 5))
 (via (at 168.5 77) (size 0.6) (drill 0.3) (layers "F.Cu" "B.Cu") (free) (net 5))
 (via (at 156.5 77) (size 0.6) (drill 0.3) (layers "F.Cu" "B.Cu") (free) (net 5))
 (via (at 166.5 83) (size 0.6) (drill 0.3) (layers "F.Cu" "B.Cu") (free) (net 5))
 (via (at 162.5 83) (size 0.6) (drill 0.3) (layers "F.Cu" "B.Cu") (free) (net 5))
 (via (at 156.5 79) (size 0.6) (drill 0.3) (layers "F.Cu" "B.Cu") (free) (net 5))
 (via (at 166.5 81) (size 0.6) (drill 0.3) (layers "F.Cu" "B.Cu") (free) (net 5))
 (via (at 156.5 81) (size 0.6) (drill 0.3) (layers "F.Cu" "B.Cu") (free) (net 5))
 (via (at 160.5 81) (size 0.6) (drill 0.3) (layers "F.Cu" "B.Cu") (free) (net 5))
 (via (at 164.5 83) (size 0.6) (drill 0.3) (layers "F.Cu" "B.Cu") (free) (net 5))
 (via (at 168.5 79) (size 0.6) (drill 0.3) (layers "F.Cu" "B.Cu") (free) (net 5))
 (via (at 158.5 83) (size 0.6) (drill 0.3) (layers "F.Cu" "B.Cu") (free) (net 5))
 (via (at 168.5 81) (size 0.6) (drill 0.3) (layers "F.Cu" "B.Cu") (free) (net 5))
 (via (at 166.5 79) (size 0.6) (drill 0.3) (layers "F.Cu" "B.Cu") (free) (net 5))
 (via (at 162.5 81) (size 0.6) (drill 0.3) (layers "F.Cu" "B.Cu") (free) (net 5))
 (via (at 158.5 81) (size 0.6) (drill 0.3) (layers "F.Cu" "B.Cu") (free) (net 5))
 (via (at 158.5 77) (size 0.6) (drill 0.3) (layers "F.Cu" "B.Cu") (free) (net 5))
 (via (at 164.5 81) (size 0.6) (drill 0.3) (layers "F.Cu" "B.Cu") (free) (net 5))
 (via (at 158.5 79) (size 0.6) (drill 0.3) (layers "F.Cu" "B.Cu") (free) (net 5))
 (via (at 168.5 83) (size 0.6) (drill 0.3) (layers "F.Cu" "B.Cu") (free) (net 5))
 (via (at 160.5 83) (size 0.6) (drill 0.3) (layers "F.Cu" "B.Cu") (free) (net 5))
 (via (at 166.5 77) (size 0.6) (drill 0.3) (layers "F.Cu" "B.Cu") (free) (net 5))
 (segment (start 151.5 82.96) (end 151.5 83.3875) (width 0.2) (layer "F.Cu") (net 9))
 (segment (start 151.5 83.3875) (end 153.1 84.9875) (width 0.2) (layer "F.Cu") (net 9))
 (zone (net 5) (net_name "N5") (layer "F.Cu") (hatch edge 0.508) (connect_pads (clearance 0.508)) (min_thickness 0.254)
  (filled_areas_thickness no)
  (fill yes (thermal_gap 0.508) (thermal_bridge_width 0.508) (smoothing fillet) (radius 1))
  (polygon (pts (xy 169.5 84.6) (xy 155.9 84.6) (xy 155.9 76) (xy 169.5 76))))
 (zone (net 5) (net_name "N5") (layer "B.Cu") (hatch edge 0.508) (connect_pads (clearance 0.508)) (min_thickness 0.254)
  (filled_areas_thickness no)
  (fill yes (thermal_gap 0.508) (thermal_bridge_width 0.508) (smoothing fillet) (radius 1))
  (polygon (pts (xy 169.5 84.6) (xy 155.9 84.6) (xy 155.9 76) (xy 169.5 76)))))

